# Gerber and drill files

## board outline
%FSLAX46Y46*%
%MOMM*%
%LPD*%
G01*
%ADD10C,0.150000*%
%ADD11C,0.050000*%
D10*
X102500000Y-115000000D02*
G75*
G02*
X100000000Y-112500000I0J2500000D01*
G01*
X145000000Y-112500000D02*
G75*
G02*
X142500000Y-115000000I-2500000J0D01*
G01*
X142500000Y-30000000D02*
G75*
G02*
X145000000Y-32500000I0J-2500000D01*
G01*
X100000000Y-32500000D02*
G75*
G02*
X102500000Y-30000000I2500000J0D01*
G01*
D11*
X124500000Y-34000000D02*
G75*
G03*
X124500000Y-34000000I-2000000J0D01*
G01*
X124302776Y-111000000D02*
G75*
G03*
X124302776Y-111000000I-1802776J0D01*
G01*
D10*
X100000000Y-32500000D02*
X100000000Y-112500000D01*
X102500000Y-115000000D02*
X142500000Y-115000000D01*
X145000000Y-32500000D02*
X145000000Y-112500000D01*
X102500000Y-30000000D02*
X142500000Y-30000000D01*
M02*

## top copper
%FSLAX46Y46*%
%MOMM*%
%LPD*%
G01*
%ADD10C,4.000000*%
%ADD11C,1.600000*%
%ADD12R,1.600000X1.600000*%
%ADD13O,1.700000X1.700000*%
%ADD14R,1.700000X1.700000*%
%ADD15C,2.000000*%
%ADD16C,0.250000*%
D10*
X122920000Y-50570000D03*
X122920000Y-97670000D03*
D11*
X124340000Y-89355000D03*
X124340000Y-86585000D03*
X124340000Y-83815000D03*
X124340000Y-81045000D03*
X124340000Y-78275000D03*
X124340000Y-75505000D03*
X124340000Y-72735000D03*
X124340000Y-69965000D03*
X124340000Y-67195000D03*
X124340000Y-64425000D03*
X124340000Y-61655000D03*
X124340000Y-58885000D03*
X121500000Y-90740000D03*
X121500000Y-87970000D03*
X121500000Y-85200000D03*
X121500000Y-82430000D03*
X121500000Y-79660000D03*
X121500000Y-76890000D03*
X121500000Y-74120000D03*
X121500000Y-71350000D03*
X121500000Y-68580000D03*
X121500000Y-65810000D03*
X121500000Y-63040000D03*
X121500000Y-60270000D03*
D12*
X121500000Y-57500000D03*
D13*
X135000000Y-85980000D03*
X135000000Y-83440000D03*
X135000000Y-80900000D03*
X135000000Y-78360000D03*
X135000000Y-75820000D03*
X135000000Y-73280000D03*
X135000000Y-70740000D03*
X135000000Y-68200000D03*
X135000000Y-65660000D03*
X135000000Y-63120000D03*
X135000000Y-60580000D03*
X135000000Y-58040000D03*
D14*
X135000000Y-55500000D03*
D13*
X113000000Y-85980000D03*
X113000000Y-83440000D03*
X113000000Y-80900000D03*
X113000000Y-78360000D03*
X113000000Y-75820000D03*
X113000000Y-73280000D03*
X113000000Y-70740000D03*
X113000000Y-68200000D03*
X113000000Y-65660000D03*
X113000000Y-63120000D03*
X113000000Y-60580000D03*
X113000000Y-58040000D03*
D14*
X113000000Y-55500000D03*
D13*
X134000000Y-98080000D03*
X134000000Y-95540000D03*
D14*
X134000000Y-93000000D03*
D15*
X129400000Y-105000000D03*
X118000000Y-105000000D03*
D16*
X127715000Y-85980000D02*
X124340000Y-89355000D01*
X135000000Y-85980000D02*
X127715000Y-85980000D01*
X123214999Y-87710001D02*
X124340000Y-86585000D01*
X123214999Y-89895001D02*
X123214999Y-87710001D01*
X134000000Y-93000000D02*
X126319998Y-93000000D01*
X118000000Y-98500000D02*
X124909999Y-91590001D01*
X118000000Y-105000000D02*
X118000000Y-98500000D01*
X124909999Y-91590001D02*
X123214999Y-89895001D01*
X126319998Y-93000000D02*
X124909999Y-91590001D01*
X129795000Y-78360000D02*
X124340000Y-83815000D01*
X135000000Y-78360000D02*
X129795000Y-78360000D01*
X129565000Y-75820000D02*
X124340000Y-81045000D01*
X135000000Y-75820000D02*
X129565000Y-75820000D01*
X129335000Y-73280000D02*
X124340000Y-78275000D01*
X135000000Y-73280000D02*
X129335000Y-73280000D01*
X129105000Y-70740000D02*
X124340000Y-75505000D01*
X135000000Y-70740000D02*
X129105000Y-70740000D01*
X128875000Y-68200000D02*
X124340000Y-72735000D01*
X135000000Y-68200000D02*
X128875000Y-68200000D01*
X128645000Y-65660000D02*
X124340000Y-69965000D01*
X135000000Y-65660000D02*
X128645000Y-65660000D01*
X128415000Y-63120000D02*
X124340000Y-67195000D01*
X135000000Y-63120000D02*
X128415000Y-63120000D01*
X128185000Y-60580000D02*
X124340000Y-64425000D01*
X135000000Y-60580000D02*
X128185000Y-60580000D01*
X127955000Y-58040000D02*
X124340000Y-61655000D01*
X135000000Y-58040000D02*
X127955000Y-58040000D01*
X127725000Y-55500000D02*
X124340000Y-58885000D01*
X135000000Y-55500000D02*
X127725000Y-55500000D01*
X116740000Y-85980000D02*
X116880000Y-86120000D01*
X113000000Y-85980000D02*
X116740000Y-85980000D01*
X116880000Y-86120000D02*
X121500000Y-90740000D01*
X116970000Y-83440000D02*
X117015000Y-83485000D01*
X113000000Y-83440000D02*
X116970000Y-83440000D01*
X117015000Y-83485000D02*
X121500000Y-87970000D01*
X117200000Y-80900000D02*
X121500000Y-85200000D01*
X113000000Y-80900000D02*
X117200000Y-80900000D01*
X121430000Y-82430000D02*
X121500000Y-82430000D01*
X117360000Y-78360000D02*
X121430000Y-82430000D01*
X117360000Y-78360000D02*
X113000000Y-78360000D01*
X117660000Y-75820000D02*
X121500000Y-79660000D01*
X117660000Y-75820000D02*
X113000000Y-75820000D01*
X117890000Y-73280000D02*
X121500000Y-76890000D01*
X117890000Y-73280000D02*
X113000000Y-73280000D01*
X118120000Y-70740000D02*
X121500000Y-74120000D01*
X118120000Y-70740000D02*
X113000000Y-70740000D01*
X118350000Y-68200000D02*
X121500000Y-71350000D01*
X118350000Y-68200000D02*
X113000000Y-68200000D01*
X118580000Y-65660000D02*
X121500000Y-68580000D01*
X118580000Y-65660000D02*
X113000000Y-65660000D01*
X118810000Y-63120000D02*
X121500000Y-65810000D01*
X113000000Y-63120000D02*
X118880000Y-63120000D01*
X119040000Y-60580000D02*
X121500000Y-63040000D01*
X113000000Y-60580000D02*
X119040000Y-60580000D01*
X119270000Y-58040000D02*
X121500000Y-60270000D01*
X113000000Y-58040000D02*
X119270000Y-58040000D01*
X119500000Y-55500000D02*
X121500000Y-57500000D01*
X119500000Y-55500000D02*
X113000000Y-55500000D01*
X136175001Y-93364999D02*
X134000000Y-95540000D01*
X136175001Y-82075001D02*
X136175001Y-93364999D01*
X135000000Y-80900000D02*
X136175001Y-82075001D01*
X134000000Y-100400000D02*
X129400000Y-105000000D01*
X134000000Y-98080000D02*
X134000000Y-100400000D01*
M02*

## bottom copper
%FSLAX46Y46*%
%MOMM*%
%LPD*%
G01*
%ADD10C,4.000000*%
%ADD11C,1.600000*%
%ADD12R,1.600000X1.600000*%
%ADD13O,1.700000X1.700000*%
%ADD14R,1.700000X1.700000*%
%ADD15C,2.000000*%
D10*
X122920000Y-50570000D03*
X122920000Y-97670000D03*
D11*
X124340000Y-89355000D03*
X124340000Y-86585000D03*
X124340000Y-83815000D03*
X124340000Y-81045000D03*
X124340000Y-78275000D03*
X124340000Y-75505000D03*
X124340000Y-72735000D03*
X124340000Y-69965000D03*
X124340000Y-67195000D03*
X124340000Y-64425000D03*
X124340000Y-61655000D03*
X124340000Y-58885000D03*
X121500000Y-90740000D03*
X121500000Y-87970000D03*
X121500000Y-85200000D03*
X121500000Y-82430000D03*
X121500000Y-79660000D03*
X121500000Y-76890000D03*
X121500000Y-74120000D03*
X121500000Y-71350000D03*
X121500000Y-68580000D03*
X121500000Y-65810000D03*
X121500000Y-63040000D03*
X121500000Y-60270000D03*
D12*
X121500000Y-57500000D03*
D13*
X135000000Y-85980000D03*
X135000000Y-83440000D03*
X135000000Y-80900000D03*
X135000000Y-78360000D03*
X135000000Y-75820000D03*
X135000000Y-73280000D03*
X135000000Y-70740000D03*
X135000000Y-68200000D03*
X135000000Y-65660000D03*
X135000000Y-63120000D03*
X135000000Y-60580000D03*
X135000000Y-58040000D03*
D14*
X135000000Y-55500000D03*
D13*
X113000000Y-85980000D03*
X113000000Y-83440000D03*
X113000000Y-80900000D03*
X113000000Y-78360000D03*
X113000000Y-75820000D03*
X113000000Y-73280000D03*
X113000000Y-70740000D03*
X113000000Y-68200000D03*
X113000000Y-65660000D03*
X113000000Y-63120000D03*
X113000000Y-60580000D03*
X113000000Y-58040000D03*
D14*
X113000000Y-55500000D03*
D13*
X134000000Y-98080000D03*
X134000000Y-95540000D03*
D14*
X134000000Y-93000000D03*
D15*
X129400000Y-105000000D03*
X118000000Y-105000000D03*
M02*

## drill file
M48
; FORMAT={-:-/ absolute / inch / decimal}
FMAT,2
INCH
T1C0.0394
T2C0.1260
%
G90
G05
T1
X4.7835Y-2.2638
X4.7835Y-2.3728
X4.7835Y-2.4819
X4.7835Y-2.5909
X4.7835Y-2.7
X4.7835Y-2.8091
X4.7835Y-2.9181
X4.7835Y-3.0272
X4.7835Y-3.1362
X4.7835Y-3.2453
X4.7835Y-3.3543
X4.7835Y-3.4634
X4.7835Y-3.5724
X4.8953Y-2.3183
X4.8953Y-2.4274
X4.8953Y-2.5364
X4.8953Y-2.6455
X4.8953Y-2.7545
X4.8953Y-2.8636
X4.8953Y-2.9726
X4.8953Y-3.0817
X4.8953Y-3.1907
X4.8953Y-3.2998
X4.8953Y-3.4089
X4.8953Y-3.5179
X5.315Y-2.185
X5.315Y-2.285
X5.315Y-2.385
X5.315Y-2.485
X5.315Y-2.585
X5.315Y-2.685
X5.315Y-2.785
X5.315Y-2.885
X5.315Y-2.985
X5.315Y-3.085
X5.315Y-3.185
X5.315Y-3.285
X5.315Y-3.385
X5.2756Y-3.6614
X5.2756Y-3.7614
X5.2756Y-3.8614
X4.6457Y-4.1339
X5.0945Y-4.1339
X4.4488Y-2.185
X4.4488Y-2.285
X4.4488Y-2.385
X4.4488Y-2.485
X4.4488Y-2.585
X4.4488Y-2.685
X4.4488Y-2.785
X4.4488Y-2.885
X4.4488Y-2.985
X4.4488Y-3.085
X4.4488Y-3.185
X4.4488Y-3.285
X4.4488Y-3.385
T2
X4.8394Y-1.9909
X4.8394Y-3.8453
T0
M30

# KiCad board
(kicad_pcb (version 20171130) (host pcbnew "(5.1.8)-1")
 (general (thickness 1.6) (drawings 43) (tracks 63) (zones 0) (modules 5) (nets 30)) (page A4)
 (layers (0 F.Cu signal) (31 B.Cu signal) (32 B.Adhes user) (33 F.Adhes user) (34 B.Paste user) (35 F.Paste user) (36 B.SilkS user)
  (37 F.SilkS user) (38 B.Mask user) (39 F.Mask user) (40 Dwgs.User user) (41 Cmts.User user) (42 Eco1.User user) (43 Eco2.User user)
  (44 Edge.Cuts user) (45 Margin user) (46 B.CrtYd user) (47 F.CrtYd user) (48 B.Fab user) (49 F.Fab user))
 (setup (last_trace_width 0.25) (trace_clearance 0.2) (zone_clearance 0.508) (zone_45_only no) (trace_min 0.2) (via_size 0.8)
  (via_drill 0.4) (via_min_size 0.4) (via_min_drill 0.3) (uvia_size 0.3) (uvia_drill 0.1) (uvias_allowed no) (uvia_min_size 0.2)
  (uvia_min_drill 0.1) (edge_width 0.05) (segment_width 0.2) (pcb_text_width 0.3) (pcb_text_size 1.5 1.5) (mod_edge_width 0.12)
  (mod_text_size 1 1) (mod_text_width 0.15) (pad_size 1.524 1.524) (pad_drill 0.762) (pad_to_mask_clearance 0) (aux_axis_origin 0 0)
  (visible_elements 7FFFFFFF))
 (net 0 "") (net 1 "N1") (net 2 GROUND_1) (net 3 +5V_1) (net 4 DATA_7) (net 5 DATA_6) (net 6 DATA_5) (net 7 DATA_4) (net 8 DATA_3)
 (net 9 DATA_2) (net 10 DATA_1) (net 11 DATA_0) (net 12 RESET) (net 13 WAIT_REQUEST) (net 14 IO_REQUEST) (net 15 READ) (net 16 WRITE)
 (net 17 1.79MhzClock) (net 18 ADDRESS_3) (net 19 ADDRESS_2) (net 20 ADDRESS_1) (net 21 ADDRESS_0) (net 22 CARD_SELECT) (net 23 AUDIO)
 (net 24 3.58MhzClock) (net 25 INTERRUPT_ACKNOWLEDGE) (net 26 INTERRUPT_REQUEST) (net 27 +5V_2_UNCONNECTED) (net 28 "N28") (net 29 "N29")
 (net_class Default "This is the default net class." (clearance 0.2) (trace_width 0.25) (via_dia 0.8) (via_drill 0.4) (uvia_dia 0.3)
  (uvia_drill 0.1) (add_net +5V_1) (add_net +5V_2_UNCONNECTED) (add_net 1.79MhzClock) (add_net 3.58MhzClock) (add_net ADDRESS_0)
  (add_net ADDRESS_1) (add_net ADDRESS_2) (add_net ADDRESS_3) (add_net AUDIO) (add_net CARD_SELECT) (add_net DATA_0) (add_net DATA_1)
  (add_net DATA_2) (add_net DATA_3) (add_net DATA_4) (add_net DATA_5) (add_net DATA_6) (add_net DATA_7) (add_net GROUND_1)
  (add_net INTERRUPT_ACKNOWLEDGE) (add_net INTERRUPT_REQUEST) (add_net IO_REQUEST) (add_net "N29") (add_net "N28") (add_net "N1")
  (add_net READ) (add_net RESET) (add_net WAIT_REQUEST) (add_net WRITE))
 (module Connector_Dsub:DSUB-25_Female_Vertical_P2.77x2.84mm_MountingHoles (layer F.Cu) (at 121.5 57.5 90)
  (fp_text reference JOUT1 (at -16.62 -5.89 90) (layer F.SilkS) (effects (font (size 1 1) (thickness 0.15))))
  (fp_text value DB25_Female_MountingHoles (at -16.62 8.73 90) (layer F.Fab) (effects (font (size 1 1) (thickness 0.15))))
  (pad 0 thru_hole circle (at 6.93 1.42 90) (size 4 4) (drill 3.2) (layers *.Cu *.Mask) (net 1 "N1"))
  (pad 0 thru_hole circle (at -40.17 1.42 90) (size 4 4) (drill 3.2) (layers *.Cu *.Mask) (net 1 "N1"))
  (pad 25 thru_hole circle (at -31.855 2.84 90) (size 1.6 1.6) (drill 1) (layers *.Cu *.Mask) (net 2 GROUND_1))
  (pad 24 thru_hole circle (at -29.085 2.84 90) (size 1.6 1.6) (drill 1) (layers *.Cu *.Mask) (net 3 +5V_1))
  (pad 23 thru_hole circle (at -26.315 2.84 90) (size 1.6 1.6) (drill 1) (layers *.Cu *.Mask) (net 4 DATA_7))
  (pad 22 thru_hole circle (at -23.545 2.84 90) (size 1.6 1.6) (drill 1) (layers *.Cu *.Mask) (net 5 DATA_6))
  (pad 21 thru_hole circle (at -20.775 2.84 90) (size 1.6 1.6) (drill 1) (layers *.Cu *.Mask) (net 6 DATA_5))
  (pad 20 thru_hole circle (at -18.005 2.84 90) (size 1.6 1.6) (drill 1) (layers *.Cu *.Mask) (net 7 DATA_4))
  (pad 19 thru_hole circle (at -15.235 2.84 90) (size 1.6 1.6) (drill 1) (layers *.Cu *.Mask) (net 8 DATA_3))
  (pad 18 thru_hole circle (at -12.465 2.84 90) (size 1.6 1.6) (drill 1) (layers *.Cu *.Mask) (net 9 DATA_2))
  (pad 17 thru_hole circle (at -9.695 2.84 90) (size 1.6 1.6) (drill 1) (layers *.Cu *.Mask) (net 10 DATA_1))
  (pad 16 thru_hole circle (at -6.925 2.84 90) (size 1.6 1.6) (drill 1) (layers *.Cu *.Mask) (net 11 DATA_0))
  (pad 15 thru_hole circle (at -4.155 2.84 90) (size 1.6 1.6) (drill 1) (layers *.Cu *.Mask) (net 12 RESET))
  (pad 14 thru_hole circle (at -1.385 2.84 90) (size 1.6 1.6) (drill 1) (layers *.Cu *.Mask) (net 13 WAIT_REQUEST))
  (pad 13 thru_hole circle (at -33.24 0 90) (size 1.6 1.6) (drill 1) (layers *.Cu *.Mask) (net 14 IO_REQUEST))
  (pad 12 thru_hole circle (at -30.47 0 90) (size 1.6 1.6) (drill 1) (layers *.Cu *.Mask) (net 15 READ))
  (pad 11 thru_hole circle (at -27.7 0 90) (size 1.6 1.6) (drill 1) (layers *.Cu *.Mask) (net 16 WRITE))
  (pad 10 thru_hole circle (at -24.93 0 90) (size 1.6 1.6) (drill 1) (layers *.Cu *.Mask) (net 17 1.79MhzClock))
  (pad 9 thru_hole circle (at -22.16 0 90) (size 1.6 1.6) (drill 1) (layers *.Cu *.Mask) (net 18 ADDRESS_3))
  (pad 8 thru_hole circle (at -19.39 0 90) (size 1.6 1.6) (drill 1) (layers *.Cu *.Mask) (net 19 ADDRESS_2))
  (pad 7 thru_hole circle (at -16.62 0 90) (size 1.6 1.6) (drill 1) (layers *.Cu *.Mask) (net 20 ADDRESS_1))
  (pad 6 thru_hole circle (at -13.85 0 90) (size 1.6 1.6) (drill 1) (layers *.Cu *.Mask) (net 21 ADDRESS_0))
  (pad 5 thru_hole circle (at -11.08 0 90) (size 1.6 1.6) (drill 1) (layers *.Cu *.Mask) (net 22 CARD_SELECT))
  (pad 4 thru_hole circle (at -8.31 0 90) (size 1.6 1.6) (drill 1) (layers *.Cu *.Mask) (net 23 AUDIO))
  (pad 3 thru_hole circle (at -5.54 0 90) (size 1.6 1.6) (drill 1) (layers *.Cu *.Mask) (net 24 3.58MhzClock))
  (pad 2 thru_hole circle (at -2.77 0 90) (size 1.6 1.6) (drill 1) (layers *.Cu *.Mask) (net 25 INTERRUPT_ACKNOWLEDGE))
  (pad 1 thru_hole rect (at 0 0 90) (size 1.6 1.6) (drill 1) (layers *.Cu *.Mask) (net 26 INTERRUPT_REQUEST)))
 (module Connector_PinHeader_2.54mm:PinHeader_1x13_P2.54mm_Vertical (layer F.Cu) (at 135 55.5)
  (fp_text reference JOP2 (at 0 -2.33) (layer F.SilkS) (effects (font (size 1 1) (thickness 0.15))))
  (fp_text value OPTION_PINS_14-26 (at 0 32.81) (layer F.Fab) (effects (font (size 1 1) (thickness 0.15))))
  (pad 13 thru_hole oval (at 0 30.48) (size 1.7 1.7) (drill 1) (layers *.Cu *.Mask) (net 2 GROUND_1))
  (pad 12 thru_hole oval (at 0 27.94) (size 1.7 1.7) (drill 1) (layers *.Cu *.Mask) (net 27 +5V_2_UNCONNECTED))
  (pad 11 thru_hole oval (at 0 25.4) (size 1.7 1.7) (drill 1) (layers *.Cu *.Mask) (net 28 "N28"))
  (pad 10 thru_hole oval (at 0 22.86) (size 1.7 1.7) (drill 1) (layers *.Cu *.Mask) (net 4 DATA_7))
  (pad 9 thru_hole oval (at 0 20.32) (size 1.7 1.7) (drill 1) (layers *.Cu *.Mask) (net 5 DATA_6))
  (pad 8 thru_hole oval (at 0 17.78) (size 1.7 1.7) (drill 1) (layers *.Cu *.Mask) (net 6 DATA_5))
  (pad 7 thru_hole oval (at 0 15.24) (size 1.7 1.7) (drill 1) (layers *.Cu *.Mask) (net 7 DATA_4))
  (pad 6 thru_hole oval (at 0 12.7) (size 1.7 1.7) (drill 1) (layers *.Cu *.Mask) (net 8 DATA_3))
  (pad 5 thru_hole oval (at 0 10.16) (size 1.7 1.7) (drill 1) (layers *.Cu *.Mask) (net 9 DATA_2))
  (pad 4 thru_hole oval (at 0 7.62) (size 1.7 1.7) (drill 1) (layers *.Cu *.Mask) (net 10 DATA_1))
  (pad 3 thru_hole oval (at 0 5.08) (size 1.7 1.7) (drill 1) (layers *.Cu *.Mask) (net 11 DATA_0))
  (pad 2 thru_hole oval (at 0 2.54) (size 1.7 1.7) (drill 1) (layers *.Cu *.Mask) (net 12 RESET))
  (pad 1 thru_hole rect (at 0 0) (size 1.7 1.7) (drill 1) (layers *.Cu *.Mask) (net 13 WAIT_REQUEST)))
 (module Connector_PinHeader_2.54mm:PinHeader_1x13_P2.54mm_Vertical (layer F.Cu) (at 113 55.5)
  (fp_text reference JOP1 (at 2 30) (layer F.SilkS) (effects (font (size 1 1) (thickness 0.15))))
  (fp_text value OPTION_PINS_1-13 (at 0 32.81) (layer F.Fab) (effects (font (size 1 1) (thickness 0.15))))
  (pad 13 thru_hole oval (at 0 30.48) (size 1.7 1.7) (drill 1) (layers *.Cu *.Mask) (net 14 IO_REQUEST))
  (pad 12 thru_hole oval (at 0 27.94) (size 1.7 1.7) (drill 1) (layers *.Cu *.Mask) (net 15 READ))
  (pad 11 thru_hole oval (at 0 25.4) (size 1.7 1.7) (drill 1) (layers *.Cu *.Mask) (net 16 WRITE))
  (pad 10 thru_hole oval (at 0 22.86) (size 1.7 1.7) (drill 1) (layers *.Cu *.Mask) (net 17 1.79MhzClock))
  (pad 9 thru_hole oval (at 0 20.32) (size 1.7 1.7) (drill 1) (layers *.Cu *.Mask) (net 18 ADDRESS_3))
  (pad 8 thru_hole oval (at 0 17.78) (size 1.7 1.7) (drill 1) (layers *.Cu *.Mask) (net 19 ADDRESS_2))
  (pad 7 thru_hole oval (at 0 15.24) (size 1.7 1.7) (drill 1) (layers *.Cu *.Mask) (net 20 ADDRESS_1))
  (pad 6 thru_hole oval (at 0 12.7) (size 1.7 1.7) (drill 1) (layers *.Cu *.Mask) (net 21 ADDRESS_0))
  (pad 5 thru_hole oval (at 0 10.16) (size 1.7 1.7) (drill 1) (layers *.Cu *.Mask) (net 22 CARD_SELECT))
  (pad 4 thru_hole oval (at 0 7.62) (size 1.7 1.7) (drill 1) (layers *.Cu *.Mask) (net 23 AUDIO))
  (pad 3 thru_hole oval (at 0 5.08) (size 1.7 1.7) (drill 1) (layers *.Cu *.Mask) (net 24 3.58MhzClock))
  (pad 2 thru_hole oval (at 0 2.54) (size 1.7 1.7) (drill 1) (layers *.Cu *.Mask) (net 25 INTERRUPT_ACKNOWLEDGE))
  (pad 1 thru_hole rect (at 0 0) (size 1.7 1.7) (drill 1) (layers *.Cu *.Mask) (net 26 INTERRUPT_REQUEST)))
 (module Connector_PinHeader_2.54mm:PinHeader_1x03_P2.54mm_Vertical (layer F.Cu) (at 134 93)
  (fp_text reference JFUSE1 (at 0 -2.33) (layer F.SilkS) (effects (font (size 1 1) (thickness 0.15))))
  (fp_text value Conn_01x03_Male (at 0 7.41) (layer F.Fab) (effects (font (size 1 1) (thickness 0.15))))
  (pad 3 thru_hole oval (at 0 5.08) (size 1.7 1.7) (drill 1) (layers *.Cu *.Mask) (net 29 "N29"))
  (pad 2 thru_hole oval (at 0 2.54) (size 1.7 1.7) (drill 1) (layers *.Cu *.Mask) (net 28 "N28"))
  (pad 1 thru_hole rect (at 0 0) (size 1.7 1.7) (drill 1) (layers *.Cu *.Mask) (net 3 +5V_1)))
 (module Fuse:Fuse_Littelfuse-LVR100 (layer F.Cu) (at 118 105)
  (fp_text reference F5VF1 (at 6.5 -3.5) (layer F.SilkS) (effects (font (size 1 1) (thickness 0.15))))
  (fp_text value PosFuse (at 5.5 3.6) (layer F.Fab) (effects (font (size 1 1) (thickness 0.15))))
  (pad 2 thru_hole circle (at 11.4 0) (size 2 2) (drill 1) (layers *.Cu *.Mask) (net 29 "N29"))
  (pad 1 thru_hole circle (at 0 0) (size 2 2) (drill 1) (layers *.Cu *.Mask) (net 3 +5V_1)))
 (gr_arc (start 102.5 112.5) (end 100 112.5) (angle -90) (layer Edge.Cuts) (width 0.15))
 (gr_arc (start 142.5 112.5) (end 142.5 115) (angle -90) (layer Edge.Cuts) (width 0.15))
 (gr_arc (start 142.5 32.5) (end 145 32.5) (angle -90) (layer Edge.Cuts) (width 0.15))
 (gr_arc (start 102.5 32.5) (end 102.5 30) (angle -90) (layer Edge.Cuts) (width 0.15))
 (gr_circle (center 122.5 34) (end 124.5 34) (layer Edge.Cuts) (width 0.05))
 (gr_circle (center 122.5 111) (end 124.302776 111) (layer Edge.Cuts) (width 0.05))
 (gr_line (start 100 32.5) (end 100 112.5) (layer Edge.Cuts) (width 0.15))
 (gr_line (start 102.5 115) (end 142.5 115) (layer Edge.Cuts) (width 0.15))
 (gr_line (start 145 32.5) (end 145 112.5) (layer Edge.Cuts) (width 0.15))
 (gr_line (start 102.5 30) (end 142.5 30) (layer Edge.Cuts) (width 0.15))
 (segment (start 127.715 85.98) (end 124.34 89.355) (width 0.25) (layer F.Cu) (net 2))
 (segment (start 135 85.98) (end 127.715 85.98) (width 0.25) (layer F.Cu) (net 2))
 (segment (start 123.214999 87.710001) (end 124.34 86.585) (width 0.25) (layer F.Cu) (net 3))
 (segment (start 123.214999 89.895001) (end 123.214999 87.710001) (width 0.25) (layer F.Cu) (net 3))
 (segment (start 134 93) (end 126.319998 93) (width 0.25) (layer F.Cu) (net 3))
 (segment (start 118 98.5) (end 124.909999 91.590001) (width 0.25) (layer F.Cu) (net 3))
 (segment (start 118 105) (end 118 98.5) (width 0.25) (layer F.Cu) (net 3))
 (segment (start 124.909999 91.590001) (end 123.214999 89.895001) (width 0.25) (layer F.Cu) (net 3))
 (segment (start 126.319998 93) (end 124.909999 91.590001) (width 0.25) (layer F.Cu) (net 3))
 (segment (start 129.795 78.36) (end 124.34 83.815) (width 0.25) (layer F.Cu) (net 4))
 (segment (start 135 78.36) (end 129.795 78.36) (width 0.25) (layer F.Cu) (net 4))
 (segment (start 129.565 75.82) (end 124.34 81.045) (width 0.25) (layer F.Cu) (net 5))
 (segment (start 135 75.82) (end 129.565 75.82) (width 0.25) (layer F.Cu) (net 5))
 (segment (start 129.335 73.28) (end 124.34 78.275) (width 0.25) (layer F.Cu) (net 6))
 (segment (start 135 73.28) (end 129.335 73.28) (width 0.25) (layer F.Cu) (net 6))
 (segment (start 129.105 70.74) (end 124.34 75.505) (width 0.25) (layer F.Cu) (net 7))
 (segment (start 135 70.74) (end 129.105 70.74) (width 0.25) (layer F.Cu) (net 7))
 (segment (start 128.875 68.2) (end 124.34 72.735) (width 0.25) (layer F.Cu) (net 8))
 (segment (start 135 68.2) (end 128.875 68.2) (width 0.25) (layer F.Cu) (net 8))
 (segment (start 128.645 65.66) (end 124.34 69.965) (width 0.25) (layer F.Cu) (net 9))
 (segment (start 135 65.66) (end 128.645 65.66) (width 0.25) (layer F.Cu) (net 9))
 (segment (start 128.415 63.12) (end 124.34 67.195) (width 0.25) (layer F.Cu) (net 10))
 (segment (start 135 63.12) (end 128.415 63.12) (width 0.25) (layer F.Cu) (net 10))
 (segment (start 128.185 60.58) (end 124.34 64.425) (width 0.25) (layer F.Cu) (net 11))
 (segment (start 135 60.58) (end 128.185 60.58) (width 0.25) (layer F.Cu) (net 11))
 (segment (start 127.955 58.04) (end 124.34 61.655) (width 0.25) (layer F.Cu) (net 12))
 (segment (start 135 58.04) (end 127.955 58.04) (width 0.25) (layer F.Cu) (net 12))
 (segment (start 127.725 55.5) (end 124.34 58.885) (width 0.25) (layer F.Cu) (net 13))
 (segment (start 135 55.5) (end 127.725 55.5) (width 0.25) (layer F.Cu) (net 13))
 (segment (start 116.74 85.98) (end 116.88 86.12) (width 0.25) (layer F.Cu) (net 14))
 (segment (start 113 85.98) (end 116.74 85.98) (width 0.25) (layer F.Cu) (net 14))
 (segment (start 116.88 86.12) (end 121.5 90.74) (width 0.25) (layer F.Cu) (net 14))
 (segment (start 116.97 83.44) (end 117.015 83.485) (width 0.25) (layer F.Cu) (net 15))
 (segment (start 113 83.44) (end 116.97 83.44) (width 0.25) (layer F.Cu) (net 15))
 (segment (start 117.015 83.485) (end 121.5 87.97) (width 0.25) (layer F.Cu) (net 15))
 (segment (start 117.2 80.9) (end 121.5 85.2) (width 0.25) (layer F.Cu) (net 16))
 (segment (start 113 80.9) (end 117.2 80.9) (width 0.25) (layer F.Cu) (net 16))
 (segment (start 121.43 82.43) (end 121.5 82.43) (width 0.25) (layer F.Cu) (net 17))
 (segment (start 117.36 78.36) (end 121.43 82.43) (width 0.25) (layer F.Cu) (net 17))
 (segment (start 117.36 78.36) (end 113 78.36) (width 0.25) (layer F.Cu) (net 17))
 (segment (start 117.66 75.82) (end 121.5 79.66) (width 0.25) (layer F.Cu) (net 18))
 (segment (start 117.66 75.82) (end 113 75.82) (width 0.25) (layer F.Cu) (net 18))
 (segment (start 117.89 73.28) (end 121.5 76.89) (width 0.25) (layer F.Cu) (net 19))
 (segment (start 117.89 73.28) (end 113 73.28) (width 0.25) (layer F.Cu) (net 19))
 (segment (start 118.12 70.74) (end 121.5 74.12) (width 0.25) (layer F.Cu) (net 20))
 (segment (start 118.12 70.74) (end 113 70.74) (width 0.25) (layer F.Cu) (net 20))
 (segment (start 118.35 68.2) (end 121.5 71.35) (width 0.25) (layer F.Cu) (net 21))
 (segment (start 118.35 68.2) (end 113 68.2) (width 0.25) (layer F.Cu) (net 21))
 (segment (start 118.58 65.66) (end 121.5 68.58) (width 0.25) (layer F.Cu) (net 22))
 (segment (start 118.58 65.66) (end 113 65.66) (width 0.25) (layer F.Cu) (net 22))
 (segment (start 118.81 63.12) (end 121.5 65.81) (width 0.25) (layer F.Cu) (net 23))
 (segment (start 113 63.12) (end 118.88 63.12) (width 0.25) (layer F.Cu) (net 23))
 (segment (start 119.04 60.58) (end 121.5 63.04) (width 0.25) (layer F.Cu) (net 24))
 (segment (start 113 60.58) (end 119.04 60.58) (width 0.25) (layer F.Cu) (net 24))
 (segment (start 119.27 58.04) (end 121.5 60.27) (width 0.25) (layer F.Cu) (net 25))
 (segment (start 113 58.04) (end 119.27 58.04) (width 0.25) (layer F.Cu) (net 25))
 (segment (start 119.5 55.5) (end 121.5 57.5) (width 0.25) (layer F.Cu) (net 26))
 (segment (start 119.5 55.5) (end 113 55.5) (width 0.25) (layer F.Cu) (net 26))
 (segment (start 136.175001 93.364999) (end 134 95.54) (width 0.25) (layer F.Cu) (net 28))
 (segment (start 136.175001 82.075001) (end 136.175001 93.364999) (width 0.25) (layer F.Cu) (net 28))
 (segment (start 135 80.9) (end 136.175001 82.075001) (width 0.25) (layer F.Cu) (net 28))
 (segment (start 134 100.4) (end 129.4 105) (width 0.25) (layer F.Cu) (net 29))
 (segment (start 134 98.08) (end 134 100.4) (width 0.25) (layer F.Cu) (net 29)))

